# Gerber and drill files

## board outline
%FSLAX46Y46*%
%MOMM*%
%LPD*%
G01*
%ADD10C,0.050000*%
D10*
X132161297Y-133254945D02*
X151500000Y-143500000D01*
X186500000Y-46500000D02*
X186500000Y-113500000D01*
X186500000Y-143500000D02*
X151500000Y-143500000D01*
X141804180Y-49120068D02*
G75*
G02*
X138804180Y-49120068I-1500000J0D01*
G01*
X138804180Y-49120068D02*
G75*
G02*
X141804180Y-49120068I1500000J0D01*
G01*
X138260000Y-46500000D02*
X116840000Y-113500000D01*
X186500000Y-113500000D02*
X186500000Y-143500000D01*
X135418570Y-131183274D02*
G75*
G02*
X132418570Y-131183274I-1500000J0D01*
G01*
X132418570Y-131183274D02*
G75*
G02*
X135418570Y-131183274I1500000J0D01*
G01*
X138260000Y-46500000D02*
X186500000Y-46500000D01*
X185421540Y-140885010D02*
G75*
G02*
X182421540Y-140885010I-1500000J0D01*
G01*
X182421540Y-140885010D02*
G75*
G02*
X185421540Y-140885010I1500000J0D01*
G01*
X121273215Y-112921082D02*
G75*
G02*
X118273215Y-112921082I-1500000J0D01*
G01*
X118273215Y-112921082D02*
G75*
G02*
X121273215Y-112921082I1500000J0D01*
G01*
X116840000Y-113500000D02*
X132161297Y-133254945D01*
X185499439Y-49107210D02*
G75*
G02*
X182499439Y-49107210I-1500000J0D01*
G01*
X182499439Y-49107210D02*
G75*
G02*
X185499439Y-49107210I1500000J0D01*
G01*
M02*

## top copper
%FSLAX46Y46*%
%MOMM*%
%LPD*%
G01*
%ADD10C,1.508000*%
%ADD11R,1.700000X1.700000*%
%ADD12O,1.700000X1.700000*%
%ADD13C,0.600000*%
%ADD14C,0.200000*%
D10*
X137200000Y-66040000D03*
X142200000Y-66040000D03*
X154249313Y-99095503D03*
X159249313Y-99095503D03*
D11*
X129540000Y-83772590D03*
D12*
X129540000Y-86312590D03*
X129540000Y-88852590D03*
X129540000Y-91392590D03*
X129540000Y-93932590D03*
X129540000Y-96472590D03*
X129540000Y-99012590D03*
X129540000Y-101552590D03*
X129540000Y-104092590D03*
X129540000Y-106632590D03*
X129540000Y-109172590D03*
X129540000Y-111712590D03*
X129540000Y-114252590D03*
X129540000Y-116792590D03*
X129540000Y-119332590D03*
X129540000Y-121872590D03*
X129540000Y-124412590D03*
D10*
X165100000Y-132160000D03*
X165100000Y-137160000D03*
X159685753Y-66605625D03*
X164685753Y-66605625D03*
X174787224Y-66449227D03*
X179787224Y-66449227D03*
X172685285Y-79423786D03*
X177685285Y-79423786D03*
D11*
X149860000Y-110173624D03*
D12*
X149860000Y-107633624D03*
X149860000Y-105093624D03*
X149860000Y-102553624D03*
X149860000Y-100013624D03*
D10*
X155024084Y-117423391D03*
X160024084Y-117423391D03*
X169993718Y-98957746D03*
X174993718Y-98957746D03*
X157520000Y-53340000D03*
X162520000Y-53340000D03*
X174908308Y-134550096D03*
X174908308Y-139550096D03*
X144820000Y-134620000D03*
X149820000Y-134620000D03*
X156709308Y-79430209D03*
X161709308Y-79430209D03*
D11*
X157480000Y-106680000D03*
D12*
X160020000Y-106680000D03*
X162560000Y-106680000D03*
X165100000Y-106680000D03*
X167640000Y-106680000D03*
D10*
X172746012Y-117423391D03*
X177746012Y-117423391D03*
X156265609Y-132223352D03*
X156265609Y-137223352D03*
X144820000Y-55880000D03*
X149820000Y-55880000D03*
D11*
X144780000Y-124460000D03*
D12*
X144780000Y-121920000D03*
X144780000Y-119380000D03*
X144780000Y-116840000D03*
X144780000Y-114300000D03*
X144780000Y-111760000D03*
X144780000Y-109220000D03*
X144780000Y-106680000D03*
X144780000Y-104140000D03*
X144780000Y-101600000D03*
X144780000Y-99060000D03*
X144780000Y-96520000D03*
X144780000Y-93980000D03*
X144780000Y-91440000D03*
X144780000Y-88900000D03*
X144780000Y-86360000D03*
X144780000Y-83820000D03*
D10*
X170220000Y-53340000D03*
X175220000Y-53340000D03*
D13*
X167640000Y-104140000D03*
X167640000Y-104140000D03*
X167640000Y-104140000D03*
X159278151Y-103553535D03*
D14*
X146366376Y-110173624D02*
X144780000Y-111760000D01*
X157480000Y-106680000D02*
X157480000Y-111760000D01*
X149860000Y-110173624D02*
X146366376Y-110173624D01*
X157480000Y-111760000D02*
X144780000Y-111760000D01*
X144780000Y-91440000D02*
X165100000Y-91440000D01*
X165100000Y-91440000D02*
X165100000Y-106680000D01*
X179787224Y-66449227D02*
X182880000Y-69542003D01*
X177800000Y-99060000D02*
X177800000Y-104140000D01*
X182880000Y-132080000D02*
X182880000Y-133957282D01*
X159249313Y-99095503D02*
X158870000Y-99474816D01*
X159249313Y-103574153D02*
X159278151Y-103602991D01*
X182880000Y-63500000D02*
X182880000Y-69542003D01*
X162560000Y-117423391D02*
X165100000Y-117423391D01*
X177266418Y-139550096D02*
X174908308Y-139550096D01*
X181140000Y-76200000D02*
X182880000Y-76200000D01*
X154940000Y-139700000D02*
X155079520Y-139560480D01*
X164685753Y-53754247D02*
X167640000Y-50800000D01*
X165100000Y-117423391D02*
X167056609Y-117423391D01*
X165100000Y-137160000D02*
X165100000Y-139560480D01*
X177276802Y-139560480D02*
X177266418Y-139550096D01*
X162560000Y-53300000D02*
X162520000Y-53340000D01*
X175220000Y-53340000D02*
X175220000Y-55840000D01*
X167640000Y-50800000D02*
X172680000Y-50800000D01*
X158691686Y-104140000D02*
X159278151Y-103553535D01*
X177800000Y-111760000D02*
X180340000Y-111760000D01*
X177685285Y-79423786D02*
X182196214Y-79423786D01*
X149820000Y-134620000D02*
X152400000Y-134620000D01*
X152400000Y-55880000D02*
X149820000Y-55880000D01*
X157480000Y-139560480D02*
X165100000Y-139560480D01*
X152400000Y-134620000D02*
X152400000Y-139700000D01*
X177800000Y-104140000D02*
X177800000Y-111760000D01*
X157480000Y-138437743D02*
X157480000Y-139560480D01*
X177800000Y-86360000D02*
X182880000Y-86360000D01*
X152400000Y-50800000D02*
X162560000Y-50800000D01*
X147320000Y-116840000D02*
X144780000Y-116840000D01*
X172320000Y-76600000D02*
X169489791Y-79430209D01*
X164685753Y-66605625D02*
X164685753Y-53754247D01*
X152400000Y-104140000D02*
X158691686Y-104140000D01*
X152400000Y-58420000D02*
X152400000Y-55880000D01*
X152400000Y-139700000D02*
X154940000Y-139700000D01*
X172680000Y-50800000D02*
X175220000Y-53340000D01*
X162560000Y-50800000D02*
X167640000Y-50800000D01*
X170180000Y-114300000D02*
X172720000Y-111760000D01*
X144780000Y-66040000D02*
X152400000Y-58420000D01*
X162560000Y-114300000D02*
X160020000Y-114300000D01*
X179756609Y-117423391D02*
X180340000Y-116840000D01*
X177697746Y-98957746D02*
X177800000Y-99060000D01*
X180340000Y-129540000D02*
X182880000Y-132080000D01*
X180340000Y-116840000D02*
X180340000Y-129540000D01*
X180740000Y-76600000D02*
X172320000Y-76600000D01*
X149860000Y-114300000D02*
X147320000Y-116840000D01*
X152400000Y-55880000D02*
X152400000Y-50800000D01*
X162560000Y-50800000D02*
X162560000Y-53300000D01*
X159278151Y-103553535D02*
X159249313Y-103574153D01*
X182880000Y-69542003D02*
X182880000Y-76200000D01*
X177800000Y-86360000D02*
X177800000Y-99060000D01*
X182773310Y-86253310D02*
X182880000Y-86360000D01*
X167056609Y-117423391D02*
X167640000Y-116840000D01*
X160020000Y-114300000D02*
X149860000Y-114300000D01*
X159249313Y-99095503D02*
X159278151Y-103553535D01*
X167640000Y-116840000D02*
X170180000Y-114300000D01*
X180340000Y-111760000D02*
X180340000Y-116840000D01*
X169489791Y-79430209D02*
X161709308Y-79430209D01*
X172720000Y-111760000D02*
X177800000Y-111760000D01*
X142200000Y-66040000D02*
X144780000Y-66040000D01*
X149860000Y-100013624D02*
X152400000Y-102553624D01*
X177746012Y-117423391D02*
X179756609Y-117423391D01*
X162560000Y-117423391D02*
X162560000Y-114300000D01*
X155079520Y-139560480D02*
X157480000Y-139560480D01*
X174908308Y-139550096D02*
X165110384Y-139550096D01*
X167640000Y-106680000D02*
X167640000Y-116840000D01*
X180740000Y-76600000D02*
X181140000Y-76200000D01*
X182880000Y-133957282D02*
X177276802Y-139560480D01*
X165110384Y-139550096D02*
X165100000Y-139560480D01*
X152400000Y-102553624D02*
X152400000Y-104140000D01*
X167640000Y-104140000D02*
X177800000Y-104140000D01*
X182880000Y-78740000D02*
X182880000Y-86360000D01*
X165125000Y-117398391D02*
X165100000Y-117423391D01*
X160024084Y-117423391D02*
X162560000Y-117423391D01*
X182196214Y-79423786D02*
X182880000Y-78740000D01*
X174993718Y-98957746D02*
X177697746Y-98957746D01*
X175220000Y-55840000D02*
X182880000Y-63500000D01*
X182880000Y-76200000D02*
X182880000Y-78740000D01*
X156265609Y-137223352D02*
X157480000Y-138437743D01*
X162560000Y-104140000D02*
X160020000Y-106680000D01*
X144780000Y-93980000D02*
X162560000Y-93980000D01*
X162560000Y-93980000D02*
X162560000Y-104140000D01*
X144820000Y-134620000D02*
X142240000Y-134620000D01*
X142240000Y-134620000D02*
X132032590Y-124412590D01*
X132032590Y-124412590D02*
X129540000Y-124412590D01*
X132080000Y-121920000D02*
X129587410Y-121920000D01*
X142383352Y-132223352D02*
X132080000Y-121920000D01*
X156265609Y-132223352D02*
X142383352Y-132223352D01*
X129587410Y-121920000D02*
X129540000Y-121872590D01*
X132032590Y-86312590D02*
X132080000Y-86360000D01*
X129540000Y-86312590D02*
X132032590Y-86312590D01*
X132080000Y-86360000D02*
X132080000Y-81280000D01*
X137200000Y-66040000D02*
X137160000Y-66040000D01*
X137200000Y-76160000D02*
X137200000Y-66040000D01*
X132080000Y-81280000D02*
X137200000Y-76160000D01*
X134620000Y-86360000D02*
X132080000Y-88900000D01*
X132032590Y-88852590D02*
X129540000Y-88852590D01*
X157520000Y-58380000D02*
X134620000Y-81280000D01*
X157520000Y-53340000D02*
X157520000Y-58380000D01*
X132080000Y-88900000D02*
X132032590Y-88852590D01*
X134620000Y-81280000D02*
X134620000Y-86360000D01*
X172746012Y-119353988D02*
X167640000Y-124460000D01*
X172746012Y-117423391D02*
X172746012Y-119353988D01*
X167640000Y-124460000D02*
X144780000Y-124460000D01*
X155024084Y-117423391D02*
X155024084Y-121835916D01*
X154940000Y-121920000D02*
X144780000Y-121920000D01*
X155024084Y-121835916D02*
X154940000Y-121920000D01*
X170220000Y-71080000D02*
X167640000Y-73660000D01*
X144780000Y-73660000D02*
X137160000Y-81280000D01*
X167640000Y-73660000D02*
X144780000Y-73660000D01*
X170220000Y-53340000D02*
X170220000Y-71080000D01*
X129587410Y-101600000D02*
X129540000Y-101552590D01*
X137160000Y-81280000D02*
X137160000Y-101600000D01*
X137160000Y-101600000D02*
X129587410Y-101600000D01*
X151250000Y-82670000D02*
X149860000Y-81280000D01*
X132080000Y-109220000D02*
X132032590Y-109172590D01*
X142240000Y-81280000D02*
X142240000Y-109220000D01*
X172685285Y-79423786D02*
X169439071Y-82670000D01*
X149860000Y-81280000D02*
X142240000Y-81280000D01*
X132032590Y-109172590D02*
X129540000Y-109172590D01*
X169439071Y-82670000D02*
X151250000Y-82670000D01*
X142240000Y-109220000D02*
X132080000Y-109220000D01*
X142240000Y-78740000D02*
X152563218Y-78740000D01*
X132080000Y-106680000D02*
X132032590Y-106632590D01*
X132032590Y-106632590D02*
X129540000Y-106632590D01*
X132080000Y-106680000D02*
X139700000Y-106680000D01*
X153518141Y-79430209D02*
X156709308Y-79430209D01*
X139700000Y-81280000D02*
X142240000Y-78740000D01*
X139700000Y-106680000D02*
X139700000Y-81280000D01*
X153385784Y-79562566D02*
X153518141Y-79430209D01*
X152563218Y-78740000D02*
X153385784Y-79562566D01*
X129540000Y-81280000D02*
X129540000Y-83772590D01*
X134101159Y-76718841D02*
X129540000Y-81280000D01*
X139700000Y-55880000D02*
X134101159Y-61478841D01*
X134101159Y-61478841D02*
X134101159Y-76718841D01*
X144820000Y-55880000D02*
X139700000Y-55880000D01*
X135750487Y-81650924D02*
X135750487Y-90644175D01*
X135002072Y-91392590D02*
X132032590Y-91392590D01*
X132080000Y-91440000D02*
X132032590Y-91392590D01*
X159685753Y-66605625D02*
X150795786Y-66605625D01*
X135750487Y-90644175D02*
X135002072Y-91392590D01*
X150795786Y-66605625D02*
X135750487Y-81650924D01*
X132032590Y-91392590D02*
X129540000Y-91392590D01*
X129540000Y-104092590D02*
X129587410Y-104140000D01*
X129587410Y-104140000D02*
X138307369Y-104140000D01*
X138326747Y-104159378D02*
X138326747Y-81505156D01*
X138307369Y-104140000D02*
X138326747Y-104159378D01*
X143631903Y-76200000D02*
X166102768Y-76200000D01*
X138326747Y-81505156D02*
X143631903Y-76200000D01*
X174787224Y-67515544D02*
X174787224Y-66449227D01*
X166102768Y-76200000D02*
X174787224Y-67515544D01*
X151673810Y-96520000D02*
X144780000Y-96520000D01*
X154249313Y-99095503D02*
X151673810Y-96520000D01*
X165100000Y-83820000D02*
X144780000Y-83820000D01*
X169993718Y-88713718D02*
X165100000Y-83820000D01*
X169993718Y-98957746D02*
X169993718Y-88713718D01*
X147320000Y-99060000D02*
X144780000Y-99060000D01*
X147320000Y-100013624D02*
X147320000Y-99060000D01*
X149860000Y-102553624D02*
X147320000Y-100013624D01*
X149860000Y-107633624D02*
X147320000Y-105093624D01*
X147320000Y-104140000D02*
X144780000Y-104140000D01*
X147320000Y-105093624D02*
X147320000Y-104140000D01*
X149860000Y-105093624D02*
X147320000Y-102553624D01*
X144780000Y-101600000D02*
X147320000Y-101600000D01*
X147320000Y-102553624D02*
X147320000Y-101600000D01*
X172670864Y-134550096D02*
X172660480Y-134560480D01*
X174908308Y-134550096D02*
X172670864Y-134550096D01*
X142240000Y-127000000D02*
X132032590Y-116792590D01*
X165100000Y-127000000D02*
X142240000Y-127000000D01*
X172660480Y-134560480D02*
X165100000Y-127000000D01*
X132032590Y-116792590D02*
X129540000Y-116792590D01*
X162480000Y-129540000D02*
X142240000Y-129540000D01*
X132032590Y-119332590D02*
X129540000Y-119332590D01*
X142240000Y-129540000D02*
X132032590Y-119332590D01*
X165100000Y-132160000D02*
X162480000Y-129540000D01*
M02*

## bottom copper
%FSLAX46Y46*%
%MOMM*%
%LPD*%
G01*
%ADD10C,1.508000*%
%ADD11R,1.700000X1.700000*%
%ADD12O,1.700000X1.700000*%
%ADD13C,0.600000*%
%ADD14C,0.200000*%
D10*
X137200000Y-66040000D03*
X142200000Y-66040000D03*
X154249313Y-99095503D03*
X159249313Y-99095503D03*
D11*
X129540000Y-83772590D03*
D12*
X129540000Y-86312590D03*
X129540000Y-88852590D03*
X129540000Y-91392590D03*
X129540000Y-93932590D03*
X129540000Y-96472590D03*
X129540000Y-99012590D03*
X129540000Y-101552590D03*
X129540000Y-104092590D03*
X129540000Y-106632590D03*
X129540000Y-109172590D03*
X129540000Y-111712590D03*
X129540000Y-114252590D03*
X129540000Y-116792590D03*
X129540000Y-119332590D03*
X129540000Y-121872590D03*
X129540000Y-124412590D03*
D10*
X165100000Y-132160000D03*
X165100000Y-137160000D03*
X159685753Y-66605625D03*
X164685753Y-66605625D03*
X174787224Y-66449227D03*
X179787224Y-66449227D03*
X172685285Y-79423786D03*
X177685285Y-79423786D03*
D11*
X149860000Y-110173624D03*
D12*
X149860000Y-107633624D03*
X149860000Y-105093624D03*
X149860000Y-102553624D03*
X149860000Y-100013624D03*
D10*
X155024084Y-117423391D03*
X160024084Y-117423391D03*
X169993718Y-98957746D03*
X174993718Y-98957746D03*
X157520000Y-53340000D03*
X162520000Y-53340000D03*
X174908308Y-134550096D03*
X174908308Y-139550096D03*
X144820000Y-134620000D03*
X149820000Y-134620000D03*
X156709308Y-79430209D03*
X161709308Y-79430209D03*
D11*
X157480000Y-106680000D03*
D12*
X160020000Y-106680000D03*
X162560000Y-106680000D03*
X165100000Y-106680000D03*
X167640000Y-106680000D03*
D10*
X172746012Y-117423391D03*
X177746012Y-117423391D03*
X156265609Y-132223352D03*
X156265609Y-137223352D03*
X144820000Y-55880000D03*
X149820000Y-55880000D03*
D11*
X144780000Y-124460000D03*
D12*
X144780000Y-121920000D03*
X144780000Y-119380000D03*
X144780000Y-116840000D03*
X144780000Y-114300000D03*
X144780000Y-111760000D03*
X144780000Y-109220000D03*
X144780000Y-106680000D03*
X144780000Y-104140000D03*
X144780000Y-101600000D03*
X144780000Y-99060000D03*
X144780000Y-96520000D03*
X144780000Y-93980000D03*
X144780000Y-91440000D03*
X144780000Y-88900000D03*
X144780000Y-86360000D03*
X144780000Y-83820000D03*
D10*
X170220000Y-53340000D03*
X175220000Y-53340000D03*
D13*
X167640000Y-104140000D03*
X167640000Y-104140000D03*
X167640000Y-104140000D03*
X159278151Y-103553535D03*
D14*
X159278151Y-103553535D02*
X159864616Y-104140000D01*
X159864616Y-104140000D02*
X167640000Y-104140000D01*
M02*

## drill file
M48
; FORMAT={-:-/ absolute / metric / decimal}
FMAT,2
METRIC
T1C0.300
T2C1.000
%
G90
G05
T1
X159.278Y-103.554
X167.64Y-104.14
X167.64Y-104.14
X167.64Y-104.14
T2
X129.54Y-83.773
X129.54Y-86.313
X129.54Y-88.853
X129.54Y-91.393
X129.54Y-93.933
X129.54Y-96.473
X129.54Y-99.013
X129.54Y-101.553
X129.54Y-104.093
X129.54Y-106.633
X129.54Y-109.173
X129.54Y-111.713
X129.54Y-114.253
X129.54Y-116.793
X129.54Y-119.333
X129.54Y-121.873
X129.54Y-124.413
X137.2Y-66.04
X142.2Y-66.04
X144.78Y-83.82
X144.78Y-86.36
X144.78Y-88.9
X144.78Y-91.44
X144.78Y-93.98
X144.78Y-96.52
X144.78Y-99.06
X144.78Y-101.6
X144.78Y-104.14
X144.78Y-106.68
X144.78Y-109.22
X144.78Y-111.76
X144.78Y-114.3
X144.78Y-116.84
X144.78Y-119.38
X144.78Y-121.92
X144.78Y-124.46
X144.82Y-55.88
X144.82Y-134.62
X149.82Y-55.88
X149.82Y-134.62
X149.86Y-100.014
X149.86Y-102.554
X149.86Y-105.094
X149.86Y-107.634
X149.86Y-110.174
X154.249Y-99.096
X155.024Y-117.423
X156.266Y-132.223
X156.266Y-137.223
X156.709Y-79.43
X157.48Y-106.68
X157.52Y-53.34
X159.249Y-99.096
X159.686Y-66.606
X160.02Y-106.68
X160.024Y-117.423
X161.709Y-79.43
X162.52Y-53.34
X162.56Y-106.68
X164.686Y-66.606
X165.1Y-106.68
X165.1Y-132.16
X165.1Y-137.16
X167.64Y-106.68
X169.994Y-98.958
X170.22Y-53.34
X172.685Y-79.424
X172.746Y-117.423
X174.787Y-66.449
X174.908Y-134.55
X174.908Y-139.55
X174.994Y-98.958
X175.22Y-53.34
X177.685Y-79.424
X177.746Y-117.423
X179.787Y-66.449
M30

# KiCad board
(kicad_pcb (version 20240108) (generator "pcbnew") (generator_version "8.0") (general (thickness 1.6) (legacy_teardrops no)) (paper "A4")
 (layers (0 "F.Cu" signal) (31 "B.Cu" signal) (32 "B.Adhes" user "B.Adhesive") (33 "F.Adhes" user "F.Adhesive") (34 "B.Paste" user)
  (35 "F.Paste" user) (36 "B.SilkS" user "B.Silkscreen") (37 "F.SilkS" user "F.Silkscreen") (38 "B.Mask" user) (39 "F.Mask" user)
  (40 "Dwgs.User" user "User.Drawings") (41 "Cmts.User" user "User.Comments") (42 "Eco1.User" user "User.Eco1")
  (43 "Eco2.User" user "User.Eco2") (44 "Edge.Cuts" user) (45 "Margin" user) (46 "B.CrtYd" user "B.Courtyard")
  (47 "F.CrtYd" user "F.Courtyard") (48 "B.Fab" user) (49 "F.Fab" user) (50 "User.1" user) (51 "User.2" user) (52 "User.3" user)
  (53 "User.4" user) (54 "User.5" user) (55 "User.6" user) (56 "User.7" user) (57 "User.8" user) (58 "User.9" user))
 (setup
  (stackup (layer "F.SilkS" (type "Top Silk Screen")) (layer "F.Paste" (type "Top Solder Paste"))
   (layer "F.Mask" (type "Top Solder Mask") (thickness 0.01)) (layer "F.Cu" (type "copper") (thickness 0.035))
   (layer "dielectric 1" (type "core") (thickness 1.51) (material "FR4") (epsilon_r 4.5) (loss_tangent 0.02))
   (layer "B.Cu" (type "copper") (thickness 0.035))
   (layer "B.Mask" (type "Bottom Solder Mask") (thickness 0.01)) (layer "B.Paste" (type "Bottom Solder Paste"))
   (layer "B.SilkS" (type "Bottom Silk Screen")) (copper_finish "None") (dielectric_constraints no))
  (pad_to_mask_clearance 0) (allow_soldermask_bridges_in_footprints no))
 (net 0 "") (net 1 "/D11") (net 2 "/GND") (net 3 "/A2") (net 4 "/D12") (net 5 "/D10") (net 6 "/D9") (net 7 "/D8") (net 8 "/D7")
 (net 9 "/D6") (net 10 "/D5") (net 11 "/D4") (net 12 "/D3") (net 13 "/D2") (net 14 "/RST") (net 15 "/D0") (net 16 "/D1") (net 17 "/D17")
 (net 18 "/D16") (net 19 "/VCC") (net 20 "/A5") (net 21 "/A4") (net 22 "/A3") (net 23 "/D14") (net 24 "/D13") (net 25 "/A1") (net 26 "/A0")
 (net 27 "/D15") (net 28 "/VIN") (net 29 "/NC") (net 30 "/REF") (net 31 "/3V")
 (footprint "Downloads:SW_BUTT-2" (layer "F.Cu") (at 139.7 66.04)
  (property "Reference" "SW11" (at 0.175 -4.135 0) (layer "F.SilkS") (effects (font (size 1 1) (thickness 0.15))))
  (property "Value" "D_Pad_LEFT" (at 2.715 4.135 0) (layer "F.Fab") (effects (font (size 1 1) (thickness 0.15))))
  (pad "1" thru_hole circle (at -2.5 0) (size 1.508 1.508) (drill 1) (layers "*.Cu" "*.Mask") (remove_unused_layers no) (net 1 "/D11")
   (solder_mask_margin 0.102))
  (pad "2" thru_hole circle (at 2.5 0) (size 1.508 1.508) (drill 1) (layers "*.Cu" "*.Mask") (remove_unused_layers no) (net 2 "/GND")
   (solder_mask_margin 0.102)))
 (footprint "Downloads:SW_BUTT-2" (layer "F.Cu") (at 156.749313 99.095503)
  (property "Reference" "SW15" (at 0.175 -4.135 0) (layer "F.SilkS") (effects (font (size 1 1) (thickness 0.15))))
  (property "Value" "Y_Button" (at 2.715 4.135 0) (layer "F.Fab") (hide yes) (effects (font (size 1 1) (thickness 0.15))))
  (pad "1" thru_hole circle (at -2.5 0) (size 1.508 1.508) (drill 1) (layers "*.Cu" "*.Mask") (remove_unused_layers no) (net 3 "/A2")
   (solder_mask_margin 0.102))
  (pad "2" thru_hole circle (at 2.5 0) (size 1.508 1.508) (drill 1) (layers "*.Cu" "*.Mask") (remove_unused_layers no) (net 2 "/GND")
   (solder_mask_margin 0.102)))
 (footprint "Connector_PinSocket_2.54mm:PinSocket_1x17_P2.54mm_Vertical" (layer "F.Cu") (at 129.54 83.77259)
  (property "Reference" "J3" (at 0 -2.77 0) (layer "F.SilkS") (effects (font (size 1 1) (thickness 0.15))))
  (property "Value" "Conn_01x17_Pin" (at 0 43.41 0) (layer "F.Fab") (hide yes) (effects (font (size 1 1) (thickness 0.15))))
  (pad "1" thru_hole rect (at 0 0) (size 1.7 1.7) (drill 1) (layers "*.Cu" "*.Mask") (remove_unused_layers no) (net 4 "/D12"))
  (pad "2" thru_hole oval (at 0 2.54) (size 1.7 1.7) (drill 1) (layers "*.Cu" "*.Mask") (remove_unused_layers no) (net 1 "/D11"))
  (pad "3" thru_hole oval (at 0 5.08) (size 1.7 1.7) (drill 1) (layers "*.Cu" "*.Mask") (remove_unused_layers no) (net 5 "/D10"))
  (pad "4" thru_hole oval (at 0 7.62) (size 1.7 1.7) (drill 1) (layers "*.Cu" "*.Mask") (remove_unused_layers no) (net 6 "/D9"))
  (pad "5" thru_hole oval (at 0 10.16) (size 1.7 1.7) (drill 1) (layers "*.Cu" "*.Mask") (remove_unused_layers no) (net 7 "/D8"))
  (pad "6" thru_hole oval (at 0 12.7) (size 1.7 1.7) (drill 1) (layers "*.Cu" "*.Mask") (remove_unused_layers no) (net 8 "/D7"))
  (pad "7" thru_hole oval (at 0 15.24) (size 1.7 1.7) (drill 1) (layers "*.Cu" "*.Mask") (remove_unused_layers no) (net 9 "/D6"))
  (pad "8" thru_hole oval (at 0 17.78) (size 1.7 1.7) (drill 1) (layers "*.Cu" "*.Mask") (remove_unused_layers no) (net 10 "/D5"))
  (pad "9" thru_hole oval (at 0 20.32) (size 1.7 1.7) (drill 1) (layers "*.Cu" "*.Mask") (remove_unused_layers no) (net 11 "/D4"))
  (pad "10" thru_hole oval (at 0 22.86) (size 1.7 1.7) (drill 1) (layers "*.Cu" "*.Mask") (remove_unused_layers no) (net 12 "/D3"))
  (pad "11" thru_hole oval (at 0 25.4) (size 1.7 1.7) (drill 1) (layers "*.Cu" "*.Mask") (remove_unused_layers no) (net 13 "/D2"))
  (pad "12" thru_hole oval (at 0 27.94) (size 1.7 1.7) (drill 1) (layers "*.Cu" "*.Mask") (remove_unused_layers no) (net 2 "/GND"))
  (pad "13" thru_hole oval (at 0 30.48) (size 1.7 1.7) (drill 1) (layers "*.Cu" "*.Mask") (remove_unused_layers no) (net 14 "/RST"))
  (pad "14" thru_hole oval (at 0 33.02) (size 1.7 1.7) (drill 1) (layers "*.Cu" "*.Mask") (remove_unused_layers no) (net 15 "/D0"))
  (pad "15" thru_hole oval (at 0 35.56) (size 1.7 1.7) (drill 1) (layers "*.Cu" "*.Mask") (remove_unused_layers no) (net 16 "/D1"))
  (pad "16" thru_hole oval (at 0 38.1) (size 1.7 1.7) (drill 1) (layers "*.Cu" "*.Mask") (remove_unused_layers no) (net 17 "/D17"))
  (pad "17" thru_hole oval (at 0 40.64) (size 1.7 1.7) (drill 1) (layers "*.Cu" "*.Mask") (remove_unused_layers no) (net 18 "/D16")))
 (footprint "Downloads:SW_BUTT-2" (layer "F.Cu") (at 165.1 134.66 -90)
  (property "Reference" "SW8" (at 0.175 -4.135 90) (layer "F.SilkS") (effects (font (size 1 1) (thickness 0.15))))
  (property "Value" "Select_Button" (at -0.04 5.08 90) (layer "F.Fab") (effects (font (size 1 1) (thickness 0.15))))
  (pad "1" thru_hole circle (at -2.5 0 270) (size 1.508 1.508) (drill 1) (layers "*.Cu" "*.Mask") (remove_unused_layers no) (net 16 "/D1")
   (solder_mask_margin 0.102))
  (pad "2" thru_hole circle (at 2.5 0 270) (size 1.508 1.508) (drill 1) (layers "*.Cu" "*.Mask") (remove_unused_layers no) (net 2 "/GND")
   (solder_mask_margin 0.102)))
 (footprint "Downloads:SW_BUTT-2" (layer "F.Cu") (at 162.185753 66.605625)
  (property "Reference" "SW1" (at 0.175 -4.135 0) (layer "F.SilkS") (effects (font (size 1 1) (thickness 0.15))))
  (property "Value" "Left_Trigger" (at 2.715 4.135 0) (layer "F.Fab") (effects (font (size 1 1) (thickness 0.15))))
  (pad "1" thru_hole circle (at -2.5 0) (size 1.508 1.508) (drill 1) (layers "*.Cu" "*.Mask") (remove_unused_layers no) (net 6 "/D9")
   (solder_mask_margin 0.102))
  (pad "2" thru_hole circle (at 2.5 0) (size 1.508 1.508) (drill 1) (layers "*.Cu" "*.Mask") (remove_unused_layers no) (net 2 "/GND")
   (solder_mask_margin 0.102)))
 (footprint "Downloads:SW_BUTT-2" (layer "F.Cu") (at 177.287224 66.449227)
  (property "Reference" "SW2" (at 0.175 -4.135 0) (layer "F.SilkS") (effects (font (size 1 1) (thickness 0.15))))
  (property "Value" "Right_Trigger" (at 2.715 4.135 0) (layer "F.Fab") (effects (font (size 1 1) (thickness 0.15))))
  (pad "1" thru_hole circle (at -2.5 0) (size 1.508 1.508) (drill 1) (layers "*.Cu" "*.Mask") (remove_unused_layers no) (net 11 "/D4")
   (solder_mask_margin 0.102))
  (pad "2" thru_hole circle (at 2.5 0) (size 1.508 1.508) (drill 1) (layers "*.Cu" "*.Mask") (remove_unused_layers no) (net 2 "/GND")
   (solder_mask_margin 0.102)))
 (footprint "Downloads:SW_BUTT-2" (layer "F.Cu") (at 175.185285 79.423786)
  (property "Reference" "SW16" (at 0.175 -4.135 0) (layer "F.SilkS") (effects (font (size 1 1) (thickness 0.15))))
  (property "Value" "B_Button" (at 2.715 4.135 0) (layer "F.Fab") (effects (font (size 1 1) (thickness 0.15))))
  (pad "1" thru_hole circle (at -2.5 0) (size 1.508 1.508) (drill 1) (layers "*.Cu" "*.Mask") (remove_unused_layers no) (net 13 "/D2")
   (solder_mask_margin 0.102))
  (pad "2" thru_hole circle (at 2.5 0) (size 1.508 1.508) (drill 1) (layers "*.Cu" "*.Mask") (remove_unused_layers no) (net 2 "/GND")
   (solder_mask_margin 0.102)))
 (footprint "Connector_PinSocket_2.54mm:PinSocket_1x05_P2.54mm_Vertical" (layer "F.Cu") (at 149.86 110.173624 180)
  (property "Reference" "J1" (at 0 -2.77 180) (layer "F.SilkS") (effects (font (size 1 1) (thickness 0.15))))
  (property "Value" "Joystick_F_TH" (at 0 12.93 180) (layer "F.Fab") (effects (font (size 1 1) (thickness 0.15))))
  (pad "1" thru_hole rect (at 0 0 180) (size 1.7 1.7) (drill 1) (layers "*.Cu" "*.Mask") (remove_unused_layers no) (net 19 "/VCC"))
  (pad "2" thru_hole oval (at 0 2.54 180) (size 1.7 1.7) (drill 1) (layers "*.Cu" "*.Mask") (remove_unused_layers no) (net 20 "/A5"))
  (pad "3" thru_hole oval (at 0 5.08 180) (size 1.7 1.7) (drill 1) (layers "*.Cu" "*.Mask") (remove_unused_layers no) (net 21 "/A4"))
  (pad "4" thru_hole oval (at 0 7.62 180) (size 1.7 1.7) (drill 1) (layers "*.Cu" "*.Mask") (remove_unused_layers no) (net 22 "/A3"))
  (pad "5" thru_hole oval (at 0 10.16 180) (size 1.7 1.7) (drill 1) (layers "*.Cu" "*.Mask") (remove_unused_layers no) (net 2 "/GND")))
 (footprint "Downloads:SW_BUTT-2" (layer "F.Cu") (at 157.524084 117.423391)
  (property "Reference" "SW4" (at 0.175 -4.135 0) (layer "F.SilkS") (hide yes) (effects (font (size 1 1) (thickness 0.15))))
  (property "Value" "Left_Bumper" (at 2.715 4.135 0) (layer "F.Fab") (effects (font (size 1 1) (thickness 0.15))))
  (pad "1" thru_hole circle (at -2.5 0) (size 1.508 1.508) (drill 1) (layers "*.Cu" "*.Mask") (remove_unused_layers no) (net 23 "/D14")
   (solder_mask_margin 0.102))
  (pad "2" thru_hole circle (at 2.5 0) (size 1.508 1.508) (drill 1) (layers "*.Cu" "*.Mask") (remove_unused_layers no) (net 2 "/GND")
   (solder_mask_margin 0.102)))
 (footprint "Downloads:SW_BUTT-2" (layer "F.Cu") (at 172.493718 98.957746)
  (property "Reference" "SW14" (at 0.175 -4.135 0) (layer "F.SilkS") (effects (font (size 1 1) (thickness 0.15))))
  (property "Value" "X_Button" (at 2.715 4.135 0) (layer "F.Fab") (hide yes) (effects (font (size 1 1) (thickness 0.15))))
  (pad "1" thru_hole circle (at -2.5 0) (size 1.508 1.508) (drill 1) (layers "*.Cu" "*.Mask") (remove_unused_layers no) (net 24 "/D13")
   (solder_mask_margin 0.102))
  (pad "2" thru_hole circle (at 2.5 0) (size 1.508 1.508) (drill 1) (layers "*.Cu" "*.Mask") (remove_unused_layers no) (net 2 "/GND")
   (solder_mask_margin 0.102)))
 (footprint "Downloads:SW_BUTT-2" (layer "F.Cu") (at 160.02 53.34)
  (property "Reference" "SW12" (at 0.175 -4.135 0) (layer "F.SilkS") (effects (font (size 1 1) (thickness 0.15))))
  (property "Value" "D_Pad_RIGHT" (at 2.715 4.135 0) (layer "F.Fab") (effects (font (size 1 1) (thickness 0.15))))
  (pad "1" thru_hole circle (at -2.5 0) (size 1.508 1.508) (drill 1) (layers "*.Cu" "*.Mask") (remove_unused_layers no) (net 5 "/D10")
   (solder_mask_margin 0.102))
  (pad "2" thru_hole circle (at 2.5 0) (size 1.508 1.508) (drill 1) (layers "*.Cu" "*.Mask") (remove_unused_layers no) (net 2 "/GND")
   (solder_mask_margin 0.102)))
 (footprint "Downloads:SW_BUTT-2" (layer "F.Cu") (at 174.908308 137.050096 -90)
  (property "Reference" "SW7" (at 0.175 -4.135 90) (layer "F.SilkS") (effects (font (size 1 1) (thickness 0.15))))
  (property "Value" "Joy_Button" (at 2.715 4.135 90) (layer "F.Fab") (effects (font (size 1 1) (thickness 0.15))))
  (pad "1" thru_hole circle (at -2.5 0 270) (size 1.508 1.508) (drill 1) (layers "*.Cu" "*.Mask") (remove_unused_layers no) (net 15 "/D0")
   (solder_mask_margin 0.102))
  (pad "2" thru_hole circle (at 2.5 0 270) (size 1.508 1.508) (drill 1) (layers "*.Cu" "*.Mask") (remove_unused_layers no) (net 2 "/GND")
   (solder_mask_margin 0.102)))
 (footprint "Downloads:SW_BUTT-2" (layer "F.Cu") (at 147.32 134.62)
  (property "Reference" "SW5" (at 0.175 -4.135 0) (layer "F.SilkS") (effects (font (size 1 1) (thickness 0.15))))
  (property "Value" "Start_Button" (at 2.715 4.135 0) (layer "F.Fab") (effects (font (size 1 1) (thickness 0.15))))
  (pad "1" thru_hole circle (at -2.5 0) (size 1.508 1.508) (drill 1) (layers "*.Cu" "*.Mask") (remove_unused_layers no) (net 18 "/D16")
   (solder_mask_margin 0.102))
  (pad "2" thru_hole circle (at 2.5 0) (size 1.508 1.508) (drill 1) (layers "*.Cu" "*.Mask") (remove_unused_layers no) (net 2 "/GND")
   (solder_mask_margin 0.102)))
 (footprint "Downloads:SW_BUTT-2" (layer "F.Cu") (at 159.209308 79.430209)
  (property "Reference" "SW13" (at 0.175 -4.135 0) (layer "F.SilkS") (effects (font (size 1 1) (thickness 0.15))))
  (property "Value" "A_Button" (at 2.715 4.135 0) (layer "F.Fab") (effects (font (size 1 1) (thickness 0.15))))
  (pad "1" thru_hole circle (at -2.5 0) (size 1.508 1.508) (drill 1) (layers "*.Cu" "*.Mask") (remove_unused_layers no) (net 12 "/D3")
   (solder_mask_margin 0.102))
  (pad "2" thru_hole circle (at 2.5 0) (size 1.508 1.508) (drill 1) (layers "*.Cu" "*.Mask") (remove_unused_layers no) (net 2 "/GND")
   (solder_mask_margin 0.102)))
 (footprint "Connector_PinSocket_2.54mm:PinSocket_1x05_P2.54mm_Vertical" (layer "F.Cu") (at 157.48 106.68 90)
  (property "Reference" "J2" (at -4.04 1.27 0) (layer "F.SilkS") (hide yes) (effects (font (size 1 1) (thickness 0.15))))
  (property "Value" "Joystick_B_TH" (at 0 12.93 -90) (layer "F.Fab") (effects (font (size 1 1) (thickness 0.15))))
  (pad "1" thru_hole rect (at 0 0 90) (size 1.7 1.7) (drill 1) (layers "*.Cu" "*.Mask") (remove_unused_layers no) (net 19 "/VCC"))
  (pad "2" thru_hole oval (at 0 2.54 90) (size 1.7 1.7) (drill 1) (layers "*.Cu" "*.Mask") (remove_unused_layers no) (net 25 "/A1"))
  (pad "3" thru_hole oval (at 0 5.08 90) (size 1.7 1.7) (drill 1) (layers "*.Cu" "*.Mask") (remove_unused_layers no) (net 10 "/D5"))
  (pad "4" thru_hole oval (at 0 7.62 90) (size 1.7 1.7) (drill 1) (layers "*.Cu" "*.Mask") (remove_unused_layers no) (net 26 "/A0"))
  (pad "5" thru_hole oval (at 0 10.16 90) (size 1.7 1.7) (drill 1) (layers "*.Cu" "*.Mask") (remove_unused_layers no) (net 2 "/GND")))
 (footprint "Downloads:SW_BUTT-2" (layer "F.Cu") (at 175.246012 117.423391)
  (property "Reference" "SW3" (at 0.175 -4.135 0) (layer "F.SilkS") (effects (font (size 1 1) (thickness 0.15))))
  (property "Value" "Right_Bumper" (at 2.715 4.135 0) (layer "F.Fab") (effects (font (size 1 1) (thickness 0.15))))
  (pad "1" thru_hole circle (at -2.5 0) (size 1.508 1.508) (drill 1) (layers "*.Cu" "*.Mask") (remove_unused_layers no) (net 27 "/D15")
   (solder_mask_margin 0.102))
  (pad "2" thru_hole circle (at 2.5 0) (size 1.508 1.508) (drill 1) (layers "*.Cu" "*.Mask") (remove_unused_layers no) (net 2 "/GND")
   (solder_mask_margin 0.102)))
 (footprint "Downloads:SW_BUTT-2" (layer "F.Cu") (at 156.265609 134.723352 -90)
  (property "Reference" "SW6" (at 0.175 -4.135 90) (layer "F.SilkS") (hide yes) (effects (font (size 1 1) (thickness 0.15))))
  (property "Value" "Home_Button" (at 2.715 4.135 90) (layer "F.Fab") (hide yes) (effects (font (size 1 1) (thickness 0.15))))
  (pad "1" thru_hole circle (at -2.5 0 270) (size 1.508 1.508) (drill 1) (layers "*.Cu" "*.Mask") (remove_unused_layers no) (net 17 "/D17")
   (solder_mask_margin 0.102))
  (pad "2" thru_hole circle (at 2.5 0 270) (size 1.508 1.508) (drill 1) (layers "*.Cu" "*.Mask") (remove_unused_layers no) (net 2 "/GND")
   (solder_mask_margin 0.102)))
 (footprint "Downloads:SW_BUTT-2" (layer "F.Cu") (at 147.32 55.88)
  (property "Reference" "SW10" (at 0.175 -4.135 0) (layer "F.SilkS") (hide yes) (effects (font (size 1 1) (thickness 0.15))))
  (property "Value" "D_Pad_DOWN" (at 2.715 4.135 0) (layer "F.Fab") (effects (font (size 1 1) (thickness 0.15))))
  (pad "1" thru_hole circle (at -2.5 0) (size 1.508 1.508) (drill 1) (layers "*.Cu" "*.Mask") (remove_unused_layers no) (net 4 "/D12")
   (solder_mask_margin 0.102))
  (pad "2" thru_hole circle (at 2.5 0) (size 1.508 1.508) (drill 1) (layers "*.Cu" "*.Mask") (remove_unused_layers no) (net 2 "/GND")
   (solder_mask_margin 0.102)))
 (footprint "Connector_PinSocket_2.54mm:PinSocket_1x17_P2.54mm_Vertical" (layer "F.Cu") (at 144.78 124.46 180)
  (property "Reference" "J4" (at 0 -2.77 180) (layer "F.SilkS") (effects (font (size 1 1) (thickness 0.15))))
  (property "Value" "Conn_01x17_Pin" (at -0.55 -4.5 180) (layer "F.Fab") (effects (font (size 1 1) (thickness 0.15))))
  (pad "1" thru_hole rect (at 0 0 180) (size 1.7 1.7) (drill 1) (layers "*.Cu" "*.Mask") (remove_unused_layers no) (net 27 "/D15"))
  (pad "2" thru_hole oval (at 0 2.54 180) (size 1.7 1.7) (drill 1) (layers "*.Cu" "*.Mask") (remove_unused_layers no) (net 23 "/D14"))
  (pad "3" thru_hole oval (at 0 5.08 180) (size 1.7 1.7) (drill 1) (layers "*.Cu" "*.Mask") (remove_unused_layers no) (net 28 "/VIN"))
  (pad "4" thru_hole oval (at 0 7.62 180) (size 1.7 1.7) (drill 1) (layers "*.Cu" "*.Mask") (remove_unused_layers no) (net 2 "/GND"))
  (pad "5" thru_hole oval (at 0 10.16 180) (size 1.7 1.7) (drill 1) (layers "*.Cu" "*.Mask") (remove_unused_layers no) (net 14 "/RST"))
  (pad "6" thru_hole oval (at 0 12.7 180) (size 1.7 1.7) (drill 1) (layers "*.Cu" "*.Mask") (remove_unused_layers no) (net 19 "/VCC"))
  (pad "7" thru_hole oval (at 0 15.24 180) (size 1.7 1.7) (drill 1) (layers "*.Cu" "*.Mask") (remove_unused_layers no) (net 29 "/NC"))
  (pad "8" thru_hole oval (at 0 17.78 180) (size 1.7 1.7) (drill 1) (layers "*.Cu" "*.Mask") (remove_unused_layers no) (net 29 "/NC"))
  (pad "9" thru_hole oval (at 0 20.32 180) (size 1.7 1.7) (drill 1) (layers "*.Cu" "*.Mask") (remove_unused_layers no) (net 20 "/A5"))
  (pad "10" thru_hole oval (at 0 22.86 180) (size 1.7 1.7) (drill 1) (layers "*.Cu" "*.Mask") (remove_unused_layers no) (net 21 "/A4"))
  (pad "11" thru_hole oval (at 0 25.4 180) (size 1.7 1.7) (drill 1) (layers "*.Cu" "*.Mask") (remove_unused_layers no) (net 22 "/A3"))
  (pad "12" thru_hole oval (at 0 27.94 180) (size 1.7 1.7) (drill 1) (layers "*.Cu" "*.Mask") (remove_unused_layers no) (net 3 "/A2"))
  (pad "13" thru_hole oval (at 0 30.48 180) (size 1.7 1.7) (drill 1) (layers "*.Cu" "*.Mask") (remove_unused_layers no) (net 25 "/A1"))
  (pad "14" thru_hole oval (at 0 33.02 180) (size 1.7 1.7) (drill 1) (layers "*.Cu" "*.Mask") (remove_unused_layers no) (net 26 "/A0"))
  (pad "15" thru_hole oval (at 0 35.56 180) (size 1.7 1.7) (drill 1) (layers "*.Cu" "*.Mask") (remove_unused_layers no) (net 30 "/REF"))
  (pad "16" thru_hole oval (at 0 38.1 180) (size 1.7 1.7) (drill 1) (layers "*.Cu" "*.Mask") (remove_unused_layers no) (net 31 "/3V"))
  (pad "17" thru_hole oval (at 0 40.64 180) (size 1.7 1.7) (drill 1) (layers "*.Cu" "*.Mask") (remove_unused_layers no) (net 24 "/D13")))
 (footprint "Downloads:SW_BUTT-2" (layer "F.Cu") (at 172.72 53.34)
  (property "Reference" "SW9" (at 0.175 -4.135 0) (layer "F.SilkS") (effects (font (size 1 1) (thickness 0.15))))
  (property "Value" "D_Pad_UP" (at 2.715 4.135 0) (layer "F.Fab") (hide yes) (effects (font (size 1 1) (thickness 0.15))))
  (pad "1" thru_hole circle (at -2.5 0) (size 1.508 1.508) (drill 1) (layers "*.Cu" "*.Mask") (remove_unused_layers no) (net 10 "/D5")
   (solder_mask_margin 0.102))
  (pad "2" thru_hole circle (at 2.5 0) (size 1.508 1.508) (drill 1) (layers "*.Cu" "*.Mask") (remove_unused_layers no) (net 2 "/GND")
   (solder_mask_margin 0.102)))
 (gr_line (start 132.161297 133.254945) (end 151.5 143.5) (stroke (width 0.05) (type default)) (layer "Edge.Cuts"))
 (gr_line (start 186.5 46.5) (end 186.5 113.5) (stroke (width 0.05) (type default)) (layer "Edge.Cuts"))
 (gr_line (start 186.5 143.5) (end 151.5 143.5) (stroke (width 0.05) (type default)) (layer "Edge.Cuts"))
 (gr_circle (center 140.30418 49.120068) (end 141.80418 49.120068) (stroke (width 0.05) (type default)) (fill none) (layer "Edge.Cuts"))
 (gr_line (start 138.26 46.5) (end 116.84 113.5) (stroke (width 0.05) (type default)) (layer "Edge.Cuts"))
 (gr_line (start 186.5 113.5) (end 186.5 143.5) (stroke (width 0.05) (type default)) (layer "Edge.Cuts"))
 (gr_circle (center 133.91857 131.183274) (end 135.41857 131.183274) (stroke (width 0.05) (type default)) (fill none) (layer "Edge.Cuts"))
 (gr_line (start 138.26 46.5) (end 186.5 46.5) (stroke (width 0.05) (type default)) (layer "Edge.Cuts"))
 (gr_circle (center 183.92154 140.88501) (end 185.42154 140.88501) (stroke (width 0.05) (type default)) (fill none) (layer "Edge.Cuts"))
 (gr_circle (center 119.773215 112.921082) (end 121.273215 112.921082) (stroke (width 0.05) (type default)) (fill none) (layer "Edge.Cuts"))
 (gr_line (start 116.84 113.5) (end 132.161297 133.254945) (stroke (width 0.05) (type default)) (layer "Edge.Cuts"))
 (gr_circle (center 183.999439 49.10721) (end 185.499439 49.10721) (stroke (width 0.05) (type default)) (fill none) (layer "Edge.Cuts"))
 (segment (start 146.366376 110.173624) (end 144.78 111.76) (width 0.2) (layer "F.Cu") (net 19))
 (segment (start 157.48 106.68) (end 157.48 111.76) (width 0.2) (layer "F.Cu") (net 19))
 (segment (start 149.86 110.173624) (end 146.366376 110.173624) (width 0.2) (layer "F.Cu") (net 19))
 (segment (start 157.48 111.76) (end 144.78 111.76) (width 0.2) (layer "F.Cu") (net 19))
 (segment (start 144.78 91.44) (end 165.1 91.44) (width 0.2) (layer "F.Cu") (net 26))
 (segment (start 165.1 91.44) (end 165.1 106.68) (width 0.2) (layer "F.Cu") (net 26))
 (segment (start 179.787224 66.449227) (end 182.88 69.542003) (width 0.2) (layer "F.Cu") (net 2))
 (segment (start 177.8 99.06) (end 177.8 104.14) (width 0.2) (layer "F.Cu") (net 2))
 (segment (start 182.88 132.08) (end 182.88 133.957282) (width 0.2) (layer "F.Cu") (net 2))
 (segment (start 159.249313 99.095503) (end 158.87 99.474816) (width 0.2) (layer "F.Cu") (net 2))
 (segment (start 159.249313 103.574153) (end 159.278151 103.602991) (width 0.2) (layer "F.Cu") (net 2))
 (segment (start 182.88 63.5) (end 182.88 69.542003) (width 0.2) (layer "F.Cu") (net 2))
 (segment (start 162.56 117.423391) (end 165.1 117.423391) (width 0.2) (layer "F.Cu") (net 2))
 (segment (start 177.266418 139.550096) (end 174.908308 139.550096) (width 0.2) (layer "F.Cu") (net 2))
 (segment (start 181.14 76.2) (end 182.88 76.2) (width 0.2) (layer "F.Cu") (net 2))
 (segment (start 154.94 139.7) (end 155.07952 139.56048) (width 0.2) (layer "F.Cu") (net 2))
 (segment (start 164.685753 53.754247) (end 167.64 50.8) (width 0.2) (layer "F.Cu") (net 2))
 (segment (start 165.1 117.423391) (end 167.056609 117.423391) (width 0.2) (layer "F.Cu") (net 2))
 (segment (start 165.1 137.16) (end 165.1 139.56048) (width 0.2) (layer "F.Cu") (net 2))
 (segment (start 177.276802 139.56048) (end 177.266418 139.550096) (width 0.2) (layer "F.Cu") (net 2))
 (segment (start 162.56 53.3) (end 162.52 53.34) (width 0.2) (layer "F.Cu") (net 2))
 (segment (start 175.22 53.34) (end 175.22 55.84) (width 0.2) (layer "F.Cu") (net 2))
 (segment (start 167.64 50.8) (end 172.68 50.8) (width 0.2) (layer "F.Cu") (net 2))
 (segment (start 158.691686 104.14) (end 159.278151 103.553535) (width 0.2) (layer "F.Cu") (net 2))
 (segment (start 177.8 111.76) (end 180.34 111.76) (width 0.2) (layer "F.Cu") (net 2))
 (segment (start 177.685285 79.423786) (end 182.196214 79.423786) (width 0.2) (layer "F.Cu") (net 2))
 (segment (start 149.82 134.62) (end 152.4 134.62) (width 0.2) (layer "F.Cu") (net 2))
 (segment (start 152.4 55.88) (end 149.82 55.88) (width 0.2) (layer "F.Cu") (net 2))
 (segment (start 157.48 139.56048) (end 165.1 139.56048) (width 0.2) (layer "F.Cu") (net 2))
 (segment (start 152.4 134.62) (end 152.4 139.7) (width 0.2) (layer "F.Cu") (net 2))
 (segment (start 177.8 104.14) (end 177.8 111.76) (width 0.2) (layer "F.Cu") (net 2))
 (segment (start 157.48 138.437743) (end 157.48 139.56048) (width 0.2) (layer "F.Cu") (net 2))
 (segment (start 177.8 86.36) (end 182.88 86.36) (width 0.2) (layer "F.Cu") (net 2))
 (segment (start 152.4 50.8) (end 162.56 50.8) (width 0.2) (layer "F.Cu") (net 2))
 (segment (start 147.32 116.84) (end 144.78 116.84) (width 0.2) (layer "F.Cu") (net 2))
 (segment (start 172.32 76.6) (end 169.489791 79.430209) (width 0.2) (layer "F.Cu") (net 2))
 (segment (start 164.685753 66.605625) (end 164.685753 53.754247) (width 0.2) (layer "F.Cu") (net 2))
 (segment (start 152.4 104.14) (end 158.691686 104.14) (width 0.2) (layer "F.Cu") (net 2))
 (segment (start 152.4 58.42) (end 152.4 55.88) (width 0.2) (layer "F.Cu") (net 2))
 (segment (start 152.4 139.7) (end 154.94 139.7) (width 0.2) (layer "F.Cu") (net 2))
 (segment (start 172.68 50.8) (end 175.22 53.34) (width 0.2) (layer "F.Cu") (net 2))
 (segment (start 162.56 50.8) (end 167.64 50.8) (width 0.2) (layer "F.Cu") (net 2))
 (segment (start 170.18 114.3) (end 172.72 111.76) (width 0.2) (layer "F.Cu") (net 2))
 (segment (start 144.78 66.04) (end 152.4 58.42) (width 0.2) (layer "F.Cu") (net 2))
 (segment (start 162.56 114.3) (end 160.02 114.3) (width 0.2) (layer "F.Cu") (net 2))
 (segment (start 179.756609 117.423391) (end 180.34 116.84) (width 0.2) (layer "F.Cu") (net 2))
 (segment (start 177.697746 98.957746) (end 177.8 99.06) (width 0.2) (layer "F.Cu") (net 2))
 (segment (start 180.34 129.54) (end 182.88 132.08) (width 0.2) (layer "F.Cu") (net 2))
 (segment (start 180.34 116.84) (end 180.34 129.54) (width 0.2) (layer "F.Cu") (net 2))
 (segment (start 180.74 76.6) (end 172.32 76.6) (width 0.2) (layer "F.Cu") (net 2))
 (segment (start 149.86 114.3) (end 147.32 116.84) (width 0.2) (layer "F.Cu") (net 2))
 (segment (start 152.4 55.88) (end 152.4 50.8) (width 0.2) (layer "F.Cu") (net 2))
 (segment (start 162.56 50.8) (end 162.56 53.3) (width 0.2) (layer "F.Cu") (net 2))
 (segment (start 159.278151 103.553535) (end 159.249313 103.574153) (width 0.2) (layer "F.Cu") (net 2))
 (segment (start 182.88 69.542003) (end 182.88 76.2) (width 0.2) (layer "F.Cu") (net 2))
 (segment (start 177.8 86.36) (end 177.8 99.06) (width 0.2) (layer "F.Cu") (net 2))
 (segment (start 182.77331 86.25331) (end 182.88 86.36) (width 0.2) (layer "F.Cu") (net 2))
 (segment (start 167.056609 117.423391) (end 167.64 116.84) (width 0.2) (layer "F.Cu") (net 2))
 (segment (start 160.02 114.3) (end 149.86 114.3) (width 0.2) (layer "F.Cu") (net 2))
 (segment (start 159.249313 99.095503) (end 159.278151 103.553535) (width 0.2) (layer "F.Cu") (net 2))
 (segment (start 167.64 116.84) (end 170.18 114.3) (width 0.2) (layer "F.Cu") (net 2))
 (segment (start 180.34 111.76) (end 180.34 116.84) (width 0.2) (layer "F.Cu") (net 2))
 (segment (start 169.489791 79.430209) (end 161.709308 79.430209) (width 0.2) (layer "F.Cu") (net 2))
 (segment (start 172.72 111.76) (end 177.8 111.76) (width 0.2) (layer "F.Cu") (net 2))
 (segment (start 142.2 66.04) (end 144.78 66.04) (width 0.2) (layer "F.Cu") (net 2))
 (segment (start 149.86 100.013624) (end 152.4 102.553624) (width 0.2) (layer "F.Cu") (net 2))
 (segment (start 177.746012 117.423391) (end 179.756609 117.423391) (width 0.2) (layer "F.Cu") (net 2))
 (segment (start 162.56 117.423391) (end 162.56 114.3) (width 0.2) (layer "F.Cu") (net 2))
 (segment (start 155.07952 139.56048) (end 157.48 139.56048) (width 0.2) (layer "F.Cu") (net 2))
 (segment (start 174.908308 139.550096) (end 165.110384 139.550096) (width 0.2) (layer "F.Cu") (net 2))
 (segment (start 167.64 106.68) (end 167.64 116.84) (width 0.2) (layer "F.Cu") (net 2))
 (segment (start 180.74 76.6) (end 181.14 76.2) (width 0.2) (layer "F.Cu") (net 2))
 (segment (start 182.88 133.957282) (end 177.276802 139.56048) (width 0.2) (layer "F.Cu") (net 2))
 (segment (start 165.110384 139.550096) (end 165.1 139.56048) (width 0.2) (layer "F.Cu") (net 2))
 (segment (start 152.4 102.553624) (end 152.4 104.14) (width 0.2) (layer "F.Cu") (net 2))
 (segment (start 167.64 104.14) (end 177.8 104.14) (width 0.2) (layer "F.Cu") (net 2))
 (segment (start 182.88 78.74) (end 182.88 86.36) (width 0.2) (layer "F.Cu") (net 2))
 (segment (start 165.125 117.398391) (end 165.1 117.423391) (width 0.2) (layer "F.Cu") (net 2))
 (segment (start 160.024084 117.423391) (end 162.56 117.423391) (width 0.2) (layer "F.Cu") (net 2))
 (segment (start 182.196214 79.423786) (end 182.88 78.74) (width 0.2) (layer "F.Cu") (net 2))
 (segment (start 174.993718 98.957746) (end 177.697746 98.957746) (width 0.2) (layer "F.Cu") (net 2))
 (segment (start 175.22 55.84) (end 182.88 63.5) (width 0.2) (layer "F.Cu") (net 2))
 (segment (start 182.88 76.2) (end 182.88 78.74) (width 0.2) (layer "F.Cu") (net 2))
 (segment (start 156.265609 137.223352) (end 157.48 138.437743) (width 0.2) (layer "F.Cu") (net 2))
 (via (at 167.64 104.14) (size 0.6) (drill 0.3) (layers "F.Cu" "B.Cu") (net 2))
 (via (at 167.64 104.14) (size 0.6) (drill 0.3) (layers "F.Cu" "B.Cu") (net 2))
 (via (at 167.64 104.14) (size 0.6) (drill 0.3) (layers "F.Cu" "B.Cu") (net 2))
 (via (at 159.278151 103.553535) (size 0.6) (drill 0.3) (layers "F.Cu" "B.Cu") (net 2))
 (segment (start 159.278151 103.553535) (end 159.864616 104.14) (width 0.2) (layer "B.Cu") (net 2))
 (segment (start 159.864616 104.14) (end 167.64 104.14) (width 0.2) (layer "B.Cu") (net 2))
 (segment (start 162.56 104.14) (end 160.02 106.68) (width 0.2) (layer "F.Cu") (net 25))
 (segment (start 144.78 93.98) (end 162.56 93.98) (width 0.2) (layer "F.Cu") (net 25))
 (segment (start 162.56 93.98) (end 162.56 104.14) (width 0.2) (layer "F.Cu") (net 25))
 (segment (start 144.82 134.62) (end 142.24 134.62) (width 0.2) (layer "F.Cu") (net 18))
 (segment (start 142.24 134.62) (end 132.03259 124.41259) (width 0.2) (layer "F.Cu") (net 18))
 (segment (start 132.03259 124.41259) (end 129.54 124.41259) (width 0.2) (layer "F.Cu") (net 18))
 (segment (start 132.08 121.92) (end 129.58741 121.92) (width 0.2) (layer "F.Cu") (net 17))
 (segment (start 142.383352 132.223352) (end 132.08 121.92) (width 0.2) (layer "F.Cu") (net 17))
 (segment (start 156.265609 132.223352) (end 142.383352 132.223352) (width 0.2) (layer "F.Cu") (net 17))
 (segment (start 129.58741 121.92) (end 129.54 121.87259) (width 0.2) (layer "F.Cu") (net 17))
 (segment (start 132.03259 86.31259) (end 132.08 86.36) (width 0.2) (layer "F.Cu") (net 1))
 (segment (start 129.54 86.31259) (end 132.03259 86.31259) (width 0.2) (layer "F.Cu") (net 1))
 (segment (start 132.08 86.36) (end 132.08 81.28) (width 0.2) (layer "F.Cu") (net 1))
 (segment (start 137.2 66.04) (end 137.16 66.04) (width 0.2) (layer "F.Cu") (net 1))
 (segment (start 137.2 76.16) (end 137.2 66.04) (width 0.2) (layer "F.Cu") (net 1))
 (segment (start 132.08 81.28) (end 137.2 76.16) (width 0.2) (layer "F.Cu") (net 1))
 (segment (start 134.62 86.36) (end 132.08 88.9) (width 0.2) (layer "F.Cu") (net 5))
 (segment (start 132.03259 88.85259) (end 129.54 88.85259) (width 0.2) (layer "F.Cu") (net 5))
 (segment (start 157.52 58.38) (end 134.62 81.28) (width 0.2) (layer "F.Cu") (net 5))
 (segment (start 157.52 53.34) (end 157.52 58.38) (width 0.2) (layer "F.Cu") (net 5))
 (segment (start 132.08 88.9) (end 132.03259 88.85259) (width 0.2) (layer "F.Cu") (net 5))
 (segment (start 134.62 81.28) (end 134.62 86.36) (width 0.2) (layer "F.Cu") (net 5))
 (segment (start 172.746012 119.353988) (end 167.64 124.46) (width 0.2) (layer "F.Cu") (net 27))
 (segment (start 172.746012 117.423391) (end 172.746012 119.353988) (width 0.2) (layer "F.Cu") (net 27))
 (segment (start 167.64 124.46) (end 144.78 124.46) (width 0.2) (layer "F.Cu") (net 27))
 (segment (start 155.024084 117.423391) (end 155.024084 121.835916) (width 0.2) (layer "F.Cu") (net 23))
 (segment (start 154.94 121.92) (end 144.78 121.92) (width 0.2) (layer "F.Cu") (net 23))
 (segment (start 155.024084 121.835916) (end 154.94 121.92) (width 0.2) (layer "F.Cu") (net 23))
 (segment (start 170.22 71.08) (end 167.64 73.66) (width 0.2) (layer "F.Cu") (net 10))
 (segment (start 144.78 73.66) (end 137.16 81.28) (width 0.2) (layer "F.Cu") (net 10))
 (segment (start 167.64 73.66) (end 144.78 73.66) (width 0.2) (layer "F.Cu") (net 10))
 (segment (start 170.22 53.34) (end 170.22 71.08) (width 0.2) (layer "F.Cu") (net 10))
 (segment (start 129.58741 101.6) (end 129.54 101.55259) (width 0.2) (layer "F.Cu") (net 10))
 (segment (start 137.16 81.28) (end 137.16 101.6) (width 0.2) (layer "F.Cu") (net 10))
 (segment (start 137.16 101.6) (end 129.58741 101.6) (width 0.2) (layer "F.Cu") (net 10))
 (segment (start 151.25 82.67) (end 149.86 81.28) (width 0.2) (layer "F.Cu") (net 13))
 (segment (start 132.08 109.22) (end 132.03259 109.17259) (width 0.2) (layer "F.Cu") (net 13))
 (segment (start 142.24 81.28) (end 142.24 109.22) (width 0.2) (layer "F.Cu") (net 13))
 (segment (start 172.685285 79.423786) (end 169.439071 82.67) (width 0.2) (layer "F.Cu") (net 13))
 (segment (start 149.86 81.28) (end 142.24 81.28) (width 0.2) (layer "F.Cu") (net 13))
 (segment (start 132.03259 109.17259) (end 129.54 109.17259) (width 0.2) (layer "F.Cu") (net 13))
 (segment (start 169.439071 82.67) (end 151.25 82.67) (width 0.2) (layer "F.Cu") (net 13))
 (segment (start 142.24 109.22) (end 132.08 109.22) (width 0.2) (layer "F.Cu") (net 13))
 (segment (start 142.24 78.74) (end 152.563218 78.74) (width 0.2) (layer "F.Cu") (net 12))
 (segment (start 132.08 106.68) (end 132.03259 106.63259) (width 0.2) (layer "F.Cu") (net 12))
 (segment (start 132.03259 106.63259) (end 129.54 106.63259) (width 0.2) (layer "F.Cu") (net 12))
 (segment (start 132.08 106.68) (end 139.7 106.68) (width 0.2) (layer "F.Cu") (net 12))
 (segment (start 153.518141 79.430209) (end 156.709308 79.430209) (width 0.2) (layer "F.Cu") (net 12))
 (segment (start 139.7 81.28) (end 142.24 78.74) (width 0.2) (layer "F.Cu") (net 12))
 (segment (start 139.7 106.68) (end 139.7 81.28) (width 0.2) (layer "F.Cu") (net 12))
 (segment (start 153.385784 79.562566) (end 153.518141 79.430209) (width 0.2) (layer "F.Cu") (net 12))
 (segment (start 152.563218 78.74) (end 153.385784 79.562566) (width 0.2) (layer "F.Cu") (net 12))
 (segment (start 129.54 81.28) (end 129.54 83.77259) (width 0.2) (layer "F.Cu") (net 4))
 (segment (start 134.101159 76.718841) (end 129.54 81.28) (width 0.2) (layer "F.Cu") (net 4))
 (segment (start 139.7 55.88) (end 134.101159 61.478841) (width 0.2) (layer "F.Cu") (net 4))
 (segment (start 134.101159 61.478841) (end 134.101159 76.718841) (width 0.2) (layer "F.Cu") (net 4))
 (segment (start 144.82 55.88) (end 139.7 55.88) (width 0.2) (layer "F.Cu") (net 4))
 (segment (start 135.750487 81.650924) (end 135.750487 90.644175) (width 0.2) (layer "F.Cu") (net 6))
 (segment (start 135.002072 91.39259) (end 132.03259 91.39259) (width 0.2) (layer "F.Cu") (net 6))
 (segment (start 132.08 91.44) (end 132.03259 91.39259) (width 0.2) (layer "F.Cu") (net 6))
 (segment (start 159.685753 66.605625) (end 150.795786 66.605625) (width 0.2) (layer "F.Cu") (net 6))
 (segment (start 135.750487 90.644175) (end 135.002072 91.39259) (width 0.2) (layer "F.Cu") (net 6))
 (segment (start 150.795786 66.605625) (end 135.750487 81.650924) (width 0.2) (layer "F.Cu") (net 6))
 (segment (start 132.03259 91.39259) (end 129.54 91.39259) (width 0.2) (layer "F.Cu") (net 6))
 (segment (start 129.54 104.09259) (end 129.58741 104.14) (width 0.2) (layer "F.Cu") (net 11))
 (segment (start 129.58741 104.14) (end 138.307369 104.14) (width 0.2) (layer "F.Cu") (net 11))
 (segment (start 138.326747 104.159378) (end 138.326747 81.505156) (width 0.2) (layer "F.Cu") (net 11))
 (segment (start 138.307369 104.14) (end 138.326747 104.159378) (width 0.2) (layer "F.Cu") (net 11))
 (segment (start 143.631903 76.2) (end 166.102768 76.2) (width 0.2) (layer "F.Cu") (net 11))
 (segment (start 138.326747 81.505156) (end 143.631903 76.2) (width 0.2) (layer "F.Cu") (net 11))
 (segment (start 174.787224 67.515544) (end 174.787224 66.449227) (width 0.2) (layer "F.Cu") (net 11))
 (segment (start 166.102768 76.2) (end 174.787224 67.515544) (width 0.2) (layer "F.Cu") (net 11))
 (segment (start 151.67381 96.52) (end 144.78 96.52) (width 0.2) (layer "F.Cu") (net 3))
 (segment (start 154.249313 99.095503) (end 151.67381 96.52) (width 0.2) (layer "F.Cu") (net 3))
 (segment (start 165.1 83.82) (end 144.78 83.82) (width 0.2) (layer "F.Cu") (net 24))
 (segment (start 169.993718 88.713718) (end 165.1 83.82) (width 0.2) (layer "F.Cu") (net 24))
 (segment (start 169.993718 98.957746) (end 169.993718 88.713718) (width 0.2) (layer "F.Cu") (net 24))
 (segment (start 147.32 99.06) (end 144.78 99.06) (width 0.2) (layer "F.Cu") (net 22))
 (segment (start 147.32 100.013624) (end 147.32 99.06) (width 0.2) (layer "F.Cu") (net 22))
 (segment (start 149.86 102.553624) (end 147.32 100.013624) (width 0.2) (layer "F.Cu") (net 22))
 (segment (start 149.86 107.633624) (end 147.32 105.093624) (width 0.2) (layer "F.Cu") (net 20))
 (segment (start 147.32 104.14) (end 144.78 104.14) (width 0.2) (layer "F.Cu") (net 20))
 (segment (start 147.32 105.093624) (end 147.32 104.14) (width 0.2) (layer "F.Cu") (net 20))
 (segment (start 149.86 105.093624) (end 147.32 102.553624) (width 0.2) (layer "F.Cu") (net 21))
 (segment (start 144.78 101.6) (end 147.32 101.6) (width 0.2) (layer "F.Cu") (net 21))
 (segment (start 147.32 102.553624) (end 147.32 101.6) (width 0.2) (layer "F.Cu") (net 21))
 (segment (start 172.670864 134.550096) (end 172.66048 134.56048) (width 0.2) (layer "F.Cu") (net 15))
 (segment (start 174.908308 134.550096) (end 172.670864 134.550096) (width 0.2) (layer "F.Cu") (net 15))
 (segment (start 142.24 127) (end 132.03259 116.79259) (width 0.2) (layer "F.Cu") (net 15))
 (segment (start 165.1 127) (end 142.24 127) (width 0.2) (layer "F.Cu") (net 15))
 (segment (start 172.66048 134.56048) (end 165.1 127) (width 0.2) (layer "F.Cu") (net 15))
 (segment (start 132.03259 116.79259) (end 129.54 116.79259) (width 0.2) (layer "F.Cu") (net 15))
 (segment (start 162.48 129.54) (end 142.24 129.54) (width 0.2) (layer "F.Cu") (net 16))
 (segment (start 132.03259 119.33259) (end 129.54 119.33259) (width 0.2) (layer "F.Cu") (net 16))
 (segment (start 142.24 129.54) (end 132.03259 119.33259) (width 0.2) (layer "F.Cu") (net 16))
 (segment (start 165.1 132.16) (end 162.48 129.54) (width 0.2) (layer "F.Cu") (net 16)))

